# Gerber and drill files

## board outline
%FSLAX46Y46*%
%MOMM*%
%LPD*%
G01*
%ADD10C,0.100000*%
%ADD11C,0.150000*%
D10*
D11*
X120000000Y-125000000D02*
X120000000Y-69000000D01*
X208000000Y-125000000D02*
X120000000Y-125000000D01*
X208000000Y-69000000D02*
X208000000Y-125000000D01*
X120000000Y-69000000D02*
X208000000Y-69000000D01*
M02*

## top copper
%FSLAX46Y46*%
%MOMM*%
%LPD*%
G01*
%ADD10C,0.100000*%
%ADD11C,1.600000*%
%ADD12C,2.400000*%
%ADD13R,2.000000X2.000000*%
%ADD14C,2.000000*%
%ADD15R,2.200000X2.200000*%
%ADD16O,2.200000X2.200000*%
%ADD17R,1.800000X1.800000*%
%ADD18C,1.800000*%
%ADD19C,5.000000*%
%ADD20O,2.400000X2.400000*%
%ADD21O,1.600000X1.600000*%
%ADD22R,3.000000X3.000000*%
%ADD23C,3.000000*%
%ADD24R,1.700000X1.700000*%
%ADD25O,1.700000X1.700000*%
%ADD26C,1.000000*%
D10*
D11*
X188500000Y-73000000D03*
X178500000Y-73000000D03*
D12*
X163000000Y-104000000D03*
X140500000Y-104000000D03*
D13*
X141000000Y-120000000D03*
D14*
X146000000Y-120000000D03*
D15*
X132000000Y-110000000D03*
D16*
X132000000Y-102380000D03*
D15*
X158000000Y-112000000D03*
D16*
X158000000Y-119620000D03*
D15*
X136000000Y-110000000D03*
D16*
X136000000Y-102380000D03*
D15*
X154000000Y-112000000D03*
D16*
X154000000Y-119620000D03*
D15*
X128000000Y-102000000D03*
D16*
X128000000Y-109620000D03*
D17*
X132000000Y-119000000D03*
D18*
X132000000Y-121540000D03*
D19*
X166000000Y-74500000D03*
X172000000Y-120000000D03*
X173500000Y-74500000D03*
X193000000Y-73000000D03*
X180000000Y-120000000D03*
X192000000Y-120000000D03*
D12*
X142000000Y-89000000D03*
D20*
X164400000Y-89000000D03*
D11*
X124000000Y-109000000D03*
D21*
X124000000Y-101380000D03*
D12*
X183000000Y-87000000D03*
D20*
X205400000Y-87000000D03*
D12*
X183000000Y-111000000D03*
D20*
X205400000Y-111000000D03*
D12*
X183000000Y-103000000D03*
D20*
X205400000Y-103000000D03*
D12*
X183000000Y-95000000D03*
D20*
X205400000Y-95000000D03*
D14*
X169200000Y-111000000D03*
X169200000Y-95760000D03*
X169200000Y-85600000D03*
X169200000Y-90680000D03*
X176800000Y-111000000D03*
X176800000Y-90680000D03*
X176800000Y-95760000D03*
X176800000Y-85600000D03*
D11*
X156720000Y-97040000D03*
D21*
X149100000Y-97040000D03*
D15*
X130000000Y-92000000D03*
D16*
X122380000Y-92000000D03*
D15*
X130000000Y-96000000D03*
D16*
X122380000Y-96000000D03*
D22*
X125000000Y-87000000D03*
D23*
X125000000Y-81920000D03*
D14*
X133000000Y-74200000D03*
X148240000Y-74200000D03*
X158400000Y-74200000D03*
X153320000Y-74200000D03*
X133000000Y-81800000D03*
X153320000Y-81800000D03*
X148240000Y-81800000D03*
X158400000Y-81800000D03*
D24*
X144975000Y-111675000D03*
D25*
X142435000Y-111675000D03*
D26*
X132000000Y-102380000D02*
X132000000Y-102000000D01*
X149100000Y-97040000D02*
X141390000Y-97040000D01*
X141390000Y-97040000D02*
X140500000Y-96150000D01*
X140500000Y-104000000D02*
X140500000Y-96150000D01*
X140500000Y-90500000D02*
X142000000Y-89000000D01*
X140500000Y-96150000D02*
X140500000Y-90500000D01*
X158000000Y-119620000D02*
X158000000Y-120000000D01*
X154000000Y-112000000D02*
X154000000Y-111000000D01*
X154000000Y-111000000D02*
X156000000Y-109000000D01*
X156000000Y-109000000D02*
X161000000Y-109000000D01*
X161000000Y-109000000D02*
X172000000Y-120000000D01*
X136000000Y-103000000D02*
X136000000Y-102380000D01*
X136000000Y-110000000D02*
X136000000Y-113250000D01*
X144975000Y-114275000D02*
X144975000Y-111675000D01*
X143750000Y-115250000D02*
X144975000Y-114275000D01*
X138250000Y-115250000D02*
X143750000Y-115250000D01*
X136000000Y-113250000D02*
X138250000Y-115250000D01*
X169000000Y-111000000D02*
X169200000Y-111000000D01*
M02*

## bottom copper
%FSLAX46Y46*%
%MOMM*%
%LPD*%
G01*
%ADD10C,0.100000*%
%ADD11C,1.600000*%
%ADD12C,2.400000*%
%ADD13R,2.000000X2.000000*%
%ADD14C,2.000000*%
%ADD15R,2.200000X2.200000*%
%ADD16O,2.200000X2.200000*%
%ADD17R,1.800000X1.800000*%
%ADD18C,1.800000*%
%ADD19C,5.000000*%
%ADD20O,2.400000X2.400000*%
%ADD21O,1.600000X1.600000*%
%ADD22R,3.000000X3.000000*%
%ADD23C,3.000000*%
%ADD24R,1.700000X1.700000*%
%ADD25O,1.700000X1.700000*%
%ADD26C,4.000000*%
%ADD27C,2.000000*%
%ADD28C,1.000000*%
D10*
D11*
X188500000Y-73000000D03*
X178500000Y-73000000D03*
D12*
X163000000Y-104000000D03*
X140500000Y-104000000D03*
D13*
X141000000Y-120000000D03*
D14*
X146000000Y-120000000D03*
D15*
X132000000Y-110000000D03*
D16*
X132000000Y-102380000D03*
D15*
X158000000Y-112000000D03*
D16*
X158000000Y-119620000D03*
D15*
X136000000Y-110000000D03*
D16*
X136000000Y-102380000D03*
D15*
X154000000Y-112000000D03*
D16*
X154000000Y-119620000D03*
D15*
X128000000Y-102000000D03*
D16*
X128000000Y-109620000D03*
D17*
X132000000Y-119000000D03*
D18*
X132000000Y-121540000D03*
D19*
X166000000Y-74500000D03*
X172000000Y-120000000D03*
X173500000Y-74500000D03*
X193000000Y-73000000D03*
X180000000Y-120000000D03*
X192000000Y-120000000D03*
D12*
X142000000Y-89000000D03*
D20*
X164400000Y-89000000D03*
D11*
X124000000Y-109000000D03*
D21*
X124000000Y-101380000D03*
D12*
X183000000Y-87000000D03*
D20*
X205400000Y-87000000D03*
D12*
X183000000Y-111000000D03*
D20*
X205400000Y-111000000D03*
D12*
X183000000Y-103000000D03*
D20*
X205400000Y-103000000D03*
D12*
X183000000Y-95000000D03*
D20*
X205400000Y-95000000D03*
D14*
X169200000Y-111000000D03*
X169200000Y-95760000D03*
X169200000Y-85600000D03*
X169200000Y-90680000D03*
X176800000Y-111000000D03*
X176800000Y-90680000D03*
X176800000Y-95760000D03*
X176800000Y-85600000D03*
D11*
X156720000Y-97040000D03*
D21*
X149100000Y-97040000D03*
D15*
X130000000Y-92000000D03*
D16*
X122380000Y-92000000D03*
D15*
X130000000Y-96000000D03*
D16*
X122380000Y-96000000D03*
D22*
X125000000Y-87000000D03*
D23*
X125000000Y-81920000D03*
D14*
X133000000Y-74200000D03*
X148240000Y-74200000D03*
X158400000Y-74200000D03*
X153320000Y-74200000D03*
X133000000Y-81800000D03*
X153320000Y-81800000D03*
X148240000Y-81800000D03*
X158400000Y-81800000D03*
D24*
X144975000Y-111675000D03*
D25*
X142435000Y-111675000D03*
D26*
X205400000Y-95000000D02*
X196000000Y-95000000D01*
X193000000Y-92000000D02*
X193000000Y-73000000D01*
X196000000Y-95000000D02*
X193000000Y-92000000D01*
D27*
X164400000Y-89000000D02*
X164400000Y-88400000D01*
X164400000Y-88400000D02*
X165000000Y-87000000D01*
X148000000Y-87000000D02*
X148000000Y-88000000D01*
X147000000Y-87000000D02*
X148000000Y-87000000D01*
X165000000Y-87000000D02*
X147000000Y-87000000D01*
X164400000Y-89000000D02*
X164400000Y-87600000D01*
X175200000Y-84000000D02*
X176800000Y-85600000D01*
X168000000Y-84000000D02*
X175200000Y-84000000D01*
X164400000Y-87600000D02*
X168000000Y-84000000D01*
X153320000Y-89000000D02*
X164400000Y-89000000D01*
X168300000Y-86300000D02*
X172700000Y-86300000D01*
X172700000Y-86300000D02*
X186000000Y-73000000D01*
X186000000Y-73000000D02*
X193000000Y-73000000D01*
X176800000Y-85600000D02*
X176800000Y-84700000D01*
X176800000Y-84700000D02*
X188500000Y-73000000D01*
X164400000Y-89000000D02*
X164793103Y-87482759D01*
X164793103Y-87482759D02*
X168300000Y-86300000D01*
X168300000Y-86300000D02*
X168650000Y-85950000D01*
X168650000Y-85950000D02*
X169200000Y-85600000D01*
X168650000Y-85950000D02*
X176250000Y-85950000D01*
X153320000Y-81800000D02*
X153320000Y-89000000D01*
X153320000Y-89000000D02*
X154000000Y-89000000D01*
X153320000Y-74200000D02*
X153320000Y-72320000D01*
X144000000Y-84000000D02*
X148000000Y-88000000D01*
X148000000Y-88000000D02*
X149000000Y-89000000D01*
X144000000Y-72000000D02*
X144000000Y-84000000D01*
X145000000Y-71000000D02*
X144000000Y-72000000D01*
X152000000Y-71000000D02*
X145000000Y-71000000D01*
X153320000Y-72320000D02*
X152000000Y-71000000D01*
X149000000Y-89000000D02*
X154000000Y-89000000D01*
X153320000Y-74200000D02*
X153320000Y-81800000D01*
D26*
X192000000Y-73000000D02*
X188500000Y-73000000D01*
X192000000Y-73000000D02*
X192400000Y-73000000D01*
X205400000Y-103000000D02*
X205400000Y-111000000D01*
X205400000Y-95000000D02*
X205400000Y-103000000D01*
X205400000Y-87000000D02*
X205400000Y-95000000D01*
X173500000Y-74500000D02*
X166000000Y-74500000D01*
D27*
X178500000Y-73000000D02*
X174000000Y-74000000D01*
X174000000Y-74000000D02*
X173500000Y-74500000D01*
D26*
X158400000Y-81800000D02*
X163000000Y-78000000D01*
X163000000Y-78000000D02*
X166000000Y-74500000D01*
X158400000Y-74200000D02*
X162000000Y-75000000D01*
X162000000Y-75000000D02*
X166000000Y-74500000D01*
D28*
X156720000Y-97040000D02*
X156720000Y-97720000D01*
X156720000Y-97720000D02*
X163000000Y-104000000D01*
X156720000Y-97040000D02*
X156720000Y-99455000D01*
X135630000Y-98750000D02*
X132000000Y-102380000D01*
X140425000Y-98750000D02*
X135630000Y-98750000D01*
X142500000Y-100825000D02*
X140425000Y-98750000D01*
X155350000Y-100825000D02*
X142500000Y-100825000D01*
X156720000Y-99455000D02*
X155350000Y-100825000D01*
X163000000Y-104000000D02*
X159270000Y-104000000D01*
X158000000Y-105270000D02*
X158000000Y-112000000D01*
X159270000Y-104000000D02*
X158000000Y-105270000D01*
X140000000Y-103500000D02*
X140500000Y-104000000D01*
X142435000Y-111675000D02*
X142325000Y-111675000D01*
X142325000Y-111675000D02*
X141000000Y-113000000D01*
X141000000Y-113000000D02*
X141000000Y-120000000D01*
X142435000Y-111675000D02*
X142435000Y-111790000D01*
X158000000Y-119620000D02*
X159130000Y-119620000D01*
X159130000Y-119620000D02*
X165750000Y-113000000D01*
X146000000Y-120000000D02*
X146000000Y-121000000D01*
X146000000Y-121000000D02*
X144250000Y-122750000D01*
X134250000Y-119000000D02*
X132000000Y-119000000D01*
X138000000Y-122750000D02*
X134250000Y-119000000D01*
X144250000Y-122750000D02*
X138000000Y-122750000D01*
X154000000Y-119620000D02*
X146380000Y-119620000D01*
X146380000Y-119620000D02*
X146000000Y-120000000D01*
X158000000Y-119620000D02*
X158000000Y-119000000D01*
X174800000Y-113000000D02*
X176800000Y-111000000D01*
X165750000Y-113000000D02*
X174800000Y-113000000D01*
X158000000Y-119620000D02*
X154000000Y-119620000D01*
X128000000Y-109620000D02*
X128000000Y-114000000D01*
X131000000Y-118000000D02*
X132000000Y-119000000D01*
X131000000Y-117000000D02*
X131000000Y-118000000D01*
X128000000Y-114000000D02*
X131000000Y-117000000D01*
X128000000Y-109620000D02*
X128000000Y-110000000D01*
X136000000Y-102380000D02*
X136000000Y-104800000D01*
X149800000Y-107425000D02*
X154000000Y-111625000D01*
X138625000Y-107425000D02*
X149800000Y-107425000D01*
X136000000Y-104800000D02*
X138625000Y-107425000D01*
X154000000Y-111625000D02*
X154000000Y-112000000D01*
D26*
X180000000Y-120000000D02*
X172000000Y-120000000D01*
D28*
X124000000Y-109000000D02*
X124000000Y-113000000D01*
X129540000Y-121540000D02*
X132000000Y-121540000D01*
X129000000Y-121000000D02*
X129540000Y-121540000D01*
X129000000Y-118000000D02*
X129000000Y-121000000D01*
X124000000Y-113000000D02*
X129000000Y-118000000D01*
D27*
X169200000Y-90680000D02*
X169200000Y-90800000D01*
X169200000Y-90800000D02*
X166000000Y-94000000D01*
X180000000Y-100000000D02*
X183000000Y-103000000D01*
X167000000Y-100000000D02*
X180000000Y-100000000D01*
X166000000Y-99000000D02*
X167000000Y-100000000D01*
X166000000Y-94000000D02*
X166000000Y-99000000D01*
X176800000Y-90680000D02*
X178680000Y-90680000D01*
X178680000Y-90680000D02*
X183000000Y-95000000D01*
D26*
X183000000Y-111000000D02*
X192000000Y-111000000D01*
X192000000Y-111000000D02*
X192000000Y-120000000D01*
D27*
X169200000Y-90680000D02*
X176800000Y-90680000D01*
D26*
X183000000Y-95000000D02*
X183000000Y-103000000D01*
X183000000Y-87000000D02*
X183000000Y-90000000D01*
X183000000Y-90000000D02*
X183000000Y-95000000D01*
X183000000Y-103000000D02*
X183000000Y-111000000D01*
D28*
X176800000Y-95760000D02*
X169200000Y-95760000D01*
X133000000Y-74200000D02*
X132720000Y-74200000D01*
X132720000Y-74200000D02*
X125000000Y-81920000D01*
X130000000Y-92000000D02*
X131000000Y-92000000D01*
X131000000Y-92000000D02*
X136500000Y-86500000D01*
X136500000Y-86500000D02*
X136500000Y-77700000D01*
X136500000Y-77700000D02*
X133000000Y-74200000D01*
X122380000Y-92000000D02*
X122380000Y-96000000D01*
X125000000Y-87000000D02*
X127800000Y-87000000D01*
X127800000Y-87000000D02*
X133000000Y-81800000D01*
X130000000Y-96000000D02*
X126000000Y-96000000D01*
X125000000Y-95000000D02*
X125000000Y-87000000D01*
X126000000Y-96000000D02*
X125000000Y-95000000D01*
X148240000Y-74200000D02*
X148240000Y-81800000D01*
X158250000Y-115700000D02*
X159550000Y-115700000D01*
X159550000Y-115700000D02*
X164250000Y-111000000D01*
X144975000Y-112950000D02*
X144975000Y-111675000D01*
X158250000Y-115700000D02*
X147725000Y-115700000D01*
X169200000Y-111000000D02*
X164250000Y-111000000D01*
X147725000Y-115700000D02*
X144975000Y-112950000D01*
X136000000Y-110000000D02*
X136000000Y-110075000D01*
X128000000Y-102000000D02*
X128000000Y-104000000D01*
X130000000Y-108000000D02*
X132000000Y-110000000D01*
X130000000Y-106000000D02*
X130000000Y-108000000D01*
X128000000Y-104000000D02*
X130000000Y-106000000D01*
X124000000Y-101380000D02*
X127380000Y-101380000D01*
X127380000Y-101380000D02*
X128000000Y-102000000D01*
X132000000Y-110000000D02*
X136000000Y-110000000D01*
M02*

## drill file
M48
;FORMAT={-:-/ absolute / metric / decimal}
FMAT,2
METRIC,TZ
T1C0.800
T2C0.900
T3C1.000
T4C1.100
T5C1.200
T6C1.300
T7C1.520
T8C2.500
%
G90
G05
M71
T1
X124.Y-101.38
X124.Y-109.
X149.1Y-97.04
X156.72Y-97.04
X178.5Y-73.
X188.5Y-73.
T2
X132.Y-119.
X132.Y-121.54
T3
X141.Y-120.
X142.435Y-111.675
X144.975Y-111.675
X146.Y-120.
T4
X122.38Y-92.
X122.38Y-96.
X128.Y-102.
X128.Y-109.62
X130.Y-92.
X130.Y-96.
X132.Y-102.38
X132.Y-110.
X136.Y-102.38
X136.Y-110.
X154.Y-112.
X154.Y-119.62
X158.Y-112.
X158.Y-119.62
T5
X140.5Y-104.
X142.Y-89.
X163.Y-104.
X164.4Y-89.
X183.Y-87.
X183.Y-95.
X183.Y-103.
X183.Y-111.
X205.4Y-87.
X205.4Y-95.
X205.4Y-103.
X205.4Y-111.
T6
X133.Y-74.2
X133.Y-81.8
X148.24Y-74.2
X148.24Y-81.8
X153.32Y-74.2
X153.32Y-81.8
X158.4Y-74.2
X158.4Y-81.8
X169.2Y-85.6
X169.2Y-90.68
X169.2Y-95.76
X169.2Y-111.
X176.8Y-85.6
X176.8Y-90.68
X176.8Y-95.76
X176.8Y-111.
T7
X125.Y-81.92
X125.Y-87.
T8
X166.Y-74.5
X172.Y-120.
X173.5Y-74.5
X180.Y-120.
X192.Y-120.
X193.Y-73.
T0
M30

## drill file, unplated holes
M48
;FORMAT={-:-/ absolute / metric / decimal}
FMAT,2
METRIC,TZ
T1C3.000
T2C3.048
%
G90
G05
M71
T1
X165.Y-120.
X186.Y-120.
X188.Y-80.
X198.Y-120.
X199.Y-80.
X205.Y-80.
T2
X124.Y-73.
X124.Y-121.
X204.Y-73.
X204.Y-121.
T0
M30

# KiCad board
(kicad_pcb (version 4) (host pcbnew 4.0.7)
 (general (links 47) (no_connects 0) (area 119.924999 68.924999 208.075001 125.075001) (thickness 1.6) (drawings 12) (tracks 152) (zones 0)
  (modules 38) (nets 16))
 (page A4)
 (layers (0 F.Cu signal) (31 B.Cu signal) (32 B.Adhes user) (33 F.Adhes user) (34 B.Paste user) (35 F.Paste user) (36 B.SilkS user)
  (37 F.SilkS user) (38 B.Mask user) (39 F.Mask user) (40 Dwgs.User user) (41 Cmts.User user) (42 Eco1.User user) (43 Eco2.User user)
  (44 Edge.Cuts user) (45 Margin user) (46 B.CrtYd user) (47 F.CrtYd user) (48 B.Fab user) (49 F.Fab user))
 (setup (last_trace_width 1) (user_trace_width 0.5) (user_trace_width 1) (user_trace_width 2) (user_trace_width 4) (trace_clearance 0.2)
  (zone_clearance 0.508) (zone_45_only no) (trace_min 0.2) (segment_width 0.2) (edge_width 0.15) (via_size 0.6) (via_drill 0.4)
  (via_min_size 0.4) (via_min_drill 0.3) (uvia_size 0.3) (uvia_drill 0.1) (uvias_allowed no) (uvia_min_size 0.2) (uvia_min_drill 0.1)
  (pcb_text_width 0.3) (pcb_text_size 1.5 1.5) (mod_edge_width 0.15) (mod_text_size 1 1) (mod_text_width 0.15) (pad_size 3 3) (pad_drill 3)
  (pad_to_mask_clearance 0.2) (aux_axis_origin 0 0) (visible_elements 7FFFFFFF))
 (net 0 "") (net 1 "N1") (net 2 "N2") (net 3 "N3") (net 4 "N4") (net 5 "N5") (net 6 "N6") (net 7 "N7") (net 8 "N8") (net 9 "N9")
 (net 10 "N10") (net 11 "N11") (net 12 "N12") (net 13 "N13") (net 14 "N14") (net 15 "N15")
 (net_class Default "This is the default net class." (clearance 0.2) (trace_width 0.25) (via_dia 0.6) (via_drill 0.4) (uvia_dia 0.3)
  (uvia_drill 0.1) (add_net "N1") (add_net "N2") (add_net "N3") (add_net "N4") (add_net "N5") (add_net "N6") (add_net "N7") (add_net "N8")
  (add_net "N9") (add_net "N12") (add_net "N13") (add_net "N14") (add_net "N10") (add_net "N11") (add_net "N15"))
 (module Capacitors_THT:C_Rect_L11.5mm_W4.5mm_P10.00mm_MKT (layer F.Cu) (at 188.5 73 180)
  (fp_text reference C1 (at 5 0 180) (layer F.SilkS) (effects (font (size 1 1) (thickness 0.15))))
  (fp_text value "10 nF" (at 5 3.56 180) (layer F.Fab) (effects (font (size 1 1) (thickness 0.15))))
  (pad 1 thru_hole circle (at 0 0 180) (size 1.6 1.6) (drill 0.8) (layers *.Cu *.Mask) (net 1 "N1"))
  (pad 2 thru_hole circle (at 10 0 180) (size 1.6 1.6) (drill 0.8) (layers *.Cu *.Mask) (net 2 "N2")))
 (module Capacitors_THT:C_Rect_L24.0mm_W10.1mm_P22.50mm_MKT (layer F.Cu) (at 163 104 180)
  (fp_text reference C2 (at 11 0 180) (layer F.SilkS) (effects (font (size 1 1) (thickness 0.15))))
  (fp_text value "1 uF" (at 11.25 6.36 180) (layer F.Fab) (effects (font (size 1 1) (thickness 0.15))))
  (pad 1 thru_hole circle (at 0 0 180) (size 2.4 2.4) (drill 1.2) (layers *.Cu *.Mask) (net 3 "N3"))
  (pad 2 thru_hole circle (at 22.5 0 180) (size 2.4 2.4) (drill 1.2) (layers *.Cu *.Mask) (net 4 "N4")))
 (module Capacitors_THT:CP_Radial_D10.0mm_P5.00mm (layer F.Cu) (at 141 120)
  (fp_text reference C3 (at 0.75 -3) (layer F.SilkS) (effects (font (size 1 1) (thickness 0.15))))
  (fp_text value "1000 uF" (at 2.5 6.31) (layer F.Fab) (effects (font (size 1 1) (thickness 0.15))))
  (pad 1 thru_hole rect (at 0 0) (size 2 2) (drill 1) (layers *.Cu *.Mask) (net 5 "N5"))
  (pad 2 thru_hole circle (at 5 0) (size 2 2) (drill 1) (layers *.Cu *.Mask) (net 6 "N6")))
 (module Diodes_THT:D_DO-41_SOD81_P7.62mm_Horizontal (layer F.Cu) (at 132 110 90)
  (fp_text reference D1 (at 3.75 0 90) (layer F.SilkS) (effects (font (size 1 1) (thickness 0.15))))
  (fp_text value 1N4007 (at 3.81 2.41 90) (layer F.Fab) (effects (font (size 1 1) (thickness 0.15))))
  (pad 1 thru_hole rect (at 0 0 90) (size 2.2 2.2) (drill 1.1) (layers *.Cu *.Mask) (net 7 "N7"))
  (pad 2 thru_hole oval (at 7.62 0 90) (size 2.2 2.2) (drill 1.1) (layers *.Cu *.Mask) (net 3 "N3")))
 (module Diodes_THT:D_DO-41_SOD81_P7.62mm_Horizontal (layer F.Cu) (at 158 112 270)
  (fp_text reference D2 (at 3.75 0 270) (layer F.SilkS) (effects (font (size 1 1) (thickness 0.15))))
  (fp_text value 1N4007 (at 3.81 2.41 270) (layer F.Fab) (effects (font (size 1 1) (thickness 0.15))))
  (pad 1 thru_hole rect (at 0 0 270) (size 2.2 2.2) (drill 1.1) (layers *.Cu *.Mask) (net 3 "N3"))
  (pad 2 thru_hole oval (at 7.62 0 270) (size 2.2 2.2) (drill 1.1) (layers *.Cu *.Mask) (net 6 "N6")))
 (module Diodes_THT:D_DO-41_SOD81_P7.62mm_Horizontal (layer F.Cu) (at 136 110 90)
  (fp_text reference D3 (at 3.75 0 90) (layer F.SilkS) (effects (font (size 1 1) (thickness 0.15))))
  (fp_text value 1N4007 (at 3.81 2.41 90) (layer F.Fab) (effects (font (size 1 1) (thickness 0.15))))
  (pad 1 thru_hole rect (at 0 0 90) (size 2.2 2.2) (drill 1.1) (layers *.Cu *.Mask) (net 7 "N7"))
  (pad 2 thru_hole oval (at 7.62 0 90) (size 2.2 2.2) (drill 1.1) (layers *.Cu *.Mask) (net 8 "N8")))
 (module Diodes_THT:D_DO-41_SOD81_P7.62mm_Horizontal (layer F.Cu) (at 154 112 270)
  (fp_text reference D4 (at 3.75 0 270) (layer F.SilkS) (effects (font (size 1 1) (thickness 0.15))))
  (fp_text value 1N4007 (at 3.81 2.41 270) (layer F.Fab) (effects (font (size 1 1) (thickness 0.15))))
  (pad 1 thru_hole rect (at 0 0 270) (size 2.2 2.2) (drill 1.1) (layers *.Cu *.Mask) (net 8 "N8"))
  (pad 2 thru_hole oval (at 7.62 0 270) (size 2.2 2.2) (drill 1.1) (layers *.Cu *.Mask) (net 6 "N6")))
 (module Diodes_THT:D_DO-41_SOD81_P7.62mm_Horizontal (layer F.Cu) (at 128 102 270)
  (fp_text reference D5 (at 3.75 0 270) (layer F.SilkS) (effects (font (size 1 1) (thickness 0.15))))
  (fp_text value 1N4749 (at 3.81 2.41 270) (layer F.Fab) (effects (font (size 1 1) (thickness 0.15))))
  (pad 1 thru_hole rect (at 0 0 270) (size 2.2 2.2) (drill 1.1) (layers *.Cu *.Mask) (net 7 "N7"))
  (pad 2 thru_hole oval (at 7.62 0 270) (size 2.2 2.2) (drill 1.1) (layers *.Cu *.Mask) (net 6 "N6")))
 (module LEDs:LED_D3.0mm (layer F.Cu) (at 132 119 270)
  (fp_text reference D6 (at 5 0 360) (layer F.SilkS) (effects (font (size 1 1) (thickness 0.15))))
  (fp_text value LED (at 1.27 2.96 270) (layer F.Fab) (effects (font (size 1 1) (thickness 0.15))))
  (pad 1 thru_hole rect (at 0 0 270) (size 1.8 1.8) (drill 0.9) (layers *.Cu *.Mask) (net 6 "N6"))
  (pad 2 thru_hole circle (at 2.54 0 270) (size 1.8 1.8) (drill 0.9) (layers *.Cu *.Mask) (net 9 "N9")))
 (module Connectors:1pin (layer F.Cu) (at 166 74.5)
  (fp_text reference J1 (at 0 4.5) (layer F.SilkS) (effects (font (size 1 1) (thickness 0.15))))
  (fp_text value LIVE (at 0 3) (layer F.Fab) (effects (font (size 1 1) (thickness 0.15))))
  (pad 1 thru_hole circle (at 0 0) (size 5 5) (drill 2.5) (layers *.Cu *.Mask) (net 2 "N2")))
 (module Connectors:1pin (layer F.Cu) (at 172 120)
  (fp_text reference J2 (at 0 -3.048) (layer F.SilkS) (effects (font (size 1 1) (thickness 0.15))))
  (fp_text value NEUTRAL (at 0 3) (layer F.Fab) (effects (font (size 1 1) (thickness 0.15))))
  (pad 1 thru_hole circle (at 0 0) (size 5 5) (drill 2.5) (layers *.Cu *.Mask) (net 8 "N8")))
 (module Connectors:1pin (layer F.Cu) (at 173.5 74.5)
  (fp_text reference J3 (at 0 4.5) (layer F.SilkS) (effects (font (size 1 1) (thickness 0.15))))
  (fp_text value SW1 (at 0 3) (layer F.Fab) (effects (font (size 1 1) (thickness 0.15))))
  (pad 1 thru_hole circle (at 0 0) (size 5 5) (drill 2.5) (layers *.Cu *.Mask) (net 2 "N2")))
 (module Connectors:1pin (layer F.Cu) (at 193 73)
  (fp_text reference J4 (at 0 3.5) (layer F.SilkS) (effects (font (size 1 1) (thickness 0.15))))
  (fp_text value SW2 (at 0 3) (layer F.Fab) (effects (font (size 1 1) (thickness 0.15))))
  (pad 1 thru_hole circle (at 0 0) (size 5 5) (drill 2.5) (layers *.Cu *.Mask) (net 1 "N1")))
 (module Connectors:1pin (layer F.Cu) (at 180 120)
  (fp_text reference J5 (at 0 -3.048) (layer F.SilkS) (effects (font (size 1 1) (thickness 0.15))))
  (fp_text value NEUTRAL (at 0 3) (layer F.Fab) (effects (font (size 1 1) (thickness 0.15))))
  (pad 1 thru_hole circle (at 0 0) (size 5 5) (drill 2.5) (layers *.Cu *.Mask) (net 8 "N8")))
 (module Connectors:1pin (layer F.Cu) (at 192 120)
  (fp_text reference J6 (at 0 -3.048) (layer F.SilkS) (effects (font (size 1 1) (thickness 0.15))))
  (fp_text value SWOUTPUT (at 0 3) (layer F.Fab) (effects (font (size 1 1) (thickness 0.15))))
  (pad 1 thru_hole circle (at 0 0) (size 5 5) (drill 2.5) (layers *.Cu *.Mask) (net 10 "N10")))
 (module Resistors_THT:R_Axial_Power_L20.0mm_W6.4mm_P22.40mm (layer F.Cu) (at 142 89)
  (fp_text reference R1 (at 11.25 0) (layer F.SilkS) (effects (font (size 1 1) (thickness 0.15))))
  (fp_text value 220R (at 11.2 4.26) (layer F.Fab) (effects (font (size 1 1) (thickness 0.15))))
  (pad 1 thru_hole circle (at 0 0) (size 2.4 2.4) (drill 1.2) (layers *.Cu *.Mask) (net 4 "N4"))
  (pad 2 thru_hole oval (at 22.4 0) (size 2.4 2.4) (drill 1.2) (layers *.Cu *.Mask) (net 1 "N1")))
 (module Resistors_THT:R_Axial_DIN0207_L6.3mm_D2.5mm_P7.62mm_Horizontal (layer F.Cu) (at 124 109 90)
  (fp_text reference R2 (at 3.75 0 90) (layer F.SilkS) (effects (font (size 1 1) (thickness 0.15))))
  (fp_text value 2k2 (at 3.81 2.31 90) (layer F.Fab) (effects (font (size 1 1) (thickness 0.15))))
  (pad 1 thru_hole circle (at 0 0 90) (size 1.6 1.6) (drill 0.8) (layers *.Cu *.Mask) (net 9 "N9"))
  (pad 2 thru_hole oval (at 7.62 0 90) (size 1.6 1.6) (drill 0.8) (layers *.Cu *.Mask) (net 7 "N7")))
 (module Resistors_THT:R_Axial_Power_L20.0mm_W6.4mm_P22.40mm (layer F.Cu) (at 183 87)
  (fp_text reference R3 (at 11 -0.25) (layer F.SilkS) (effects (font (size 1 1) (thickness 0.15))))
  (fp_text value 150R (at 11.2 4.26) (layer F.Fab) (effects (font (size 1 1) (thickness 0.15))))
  (pad 1 thru_hole circle (at 0 0) (size 2.4 2.4) (drill 1.2) (layers *.Cu *.Mask) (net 10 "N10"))
  (pad 2 thru_hole oval (at 22.4 0) (size 2.4 2.4) (drill 1.2) (layers *.Cu *.Mask) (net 1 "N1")))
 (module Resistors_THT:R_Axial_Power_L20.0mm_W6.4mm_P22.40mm (layer F.Cu) (at 183 111)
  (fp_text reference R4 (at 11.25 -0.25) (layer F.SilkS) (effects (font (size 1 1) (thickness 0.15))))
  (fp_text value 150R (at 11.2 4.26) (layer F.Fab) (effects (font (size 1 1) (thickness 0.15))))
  (pad 1 thru_hole circle (at 0 0) (size 2.4 2.4) (drill 1.2) (layers *.Cu *.Mask) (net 10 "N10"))
  (pad 2 thru_hole oval (at 22.4 0) (size 2.4 2.4) (drill 1.2) (layers *.Cu *.Mask) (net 1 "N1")))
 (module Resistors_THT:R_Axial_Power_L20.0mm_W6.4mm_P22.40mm (layer F.Cu) (at 183 103)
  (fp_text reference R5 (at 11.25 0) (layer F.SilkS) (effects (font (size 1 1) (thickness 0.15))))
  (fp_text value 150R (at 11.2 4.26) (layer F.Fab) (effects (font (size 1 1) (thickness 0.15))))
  (pad 1 thru_hole circle (at 0 0) (size 2.4 2.4) (drill 1.2) (layers *.Cu *.Mask) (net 10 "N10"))
  (pad 2 thru_hole oval (at 22.4 0) (size 2.4 2.4) (drill 1.2) (layers *.Cu *.Mask) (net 1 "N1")))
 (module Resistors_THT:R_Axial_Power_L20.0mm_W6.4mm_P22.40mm (layer F.Cu) (at 183 95)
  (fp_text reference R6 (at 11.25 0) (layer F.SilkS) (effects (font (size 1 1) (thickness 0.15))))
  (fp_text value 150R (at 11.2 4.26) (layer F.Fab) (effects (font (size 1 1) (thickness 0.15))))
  (pad 1 thru_hole circle (at 0 0) (size 2.4 2.4) (drill 1.2) (layers *.Cu *.Mask) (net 10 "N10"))
  (pad 2 thru_hole oval (at 22.4 0) (size 2.4 2.4) (drill 1.2) (layers *.Cu *.Mask) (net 1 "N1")))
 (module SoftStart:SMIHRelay (layer F.Cu) (at 173 101 90)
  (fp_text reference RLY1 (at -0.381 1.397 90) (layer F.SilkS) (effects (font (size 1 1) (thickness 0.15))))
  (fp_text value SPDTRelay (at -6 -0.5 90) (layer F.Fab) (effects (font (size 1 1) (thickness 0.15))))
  (pad 4 thru_hole circle (at -10 -3.8 90) (size 2 2) (drill 1.3) (layers *.Cu *.Mask) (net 7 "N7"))
  (pad 2 thru_hole circle (at 5.24 -3.8 90) (size 2 2) (drill 1.3) (layers *.Cu *.Mask) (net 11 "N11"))
  (pad 3 thru_hole circle (at 15.4 -3.8 90) (size 2 2) (drill 1.3) (layers *.Cu *.Mask) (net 1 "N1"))
  (pad 1 thru_hole circle (at 10.32 -3.8 90) (size 2 2) (drill 1.3) (layers *.Cu *.Mask) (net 10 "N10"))
  (pad 5 thru_hole circle (at -10 3.8 90) (size 2 2) (drill 1.3) (layers *.Cu *.Mask) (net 6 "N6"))
  (pad 1 thru_hole circle (at 10.32 3.8 90) (size 2 2) (drill 1.3) (layers *.Cu *.Mask) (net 10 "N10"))
  (pad 2 thru_hole circle (at 5.24 3.8 90) (size 2 2) (drill 1.3) (layers *.Cu *.Mask) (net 11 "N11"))
  (pad 3 thru_hole circle (at 15.4 3.8 90) (size 2 2) (drill 1.3) (layers *.Cu *.Mask) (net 1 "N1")))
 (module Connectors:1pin (layer F.Cu) (at 204 121)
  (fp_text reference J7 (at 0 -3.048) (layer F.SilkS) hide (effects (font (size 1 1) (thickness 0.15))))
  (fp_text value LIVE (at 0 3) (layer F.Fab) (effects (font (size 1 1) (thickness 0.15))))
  (pad "" np_thru_hole circle (at 0 0) (size 3.048 3.048) (drill 3.048) (layers *.Cu *.Mask)))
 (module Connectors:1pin (layer F.Cu) (at 204 73)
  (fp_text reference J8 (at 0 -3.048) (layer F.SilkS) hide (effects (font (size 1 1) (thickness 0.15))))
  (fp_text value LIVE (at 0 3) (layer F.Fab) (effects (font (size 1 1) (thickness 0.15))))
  (pad "" np_thru_hole circle (at 0 0) (size 3.048 3.048) (drill 3.048) (layers *.Cu *.Mask)))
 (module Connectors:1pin (layer F.Cu) (at 124 73)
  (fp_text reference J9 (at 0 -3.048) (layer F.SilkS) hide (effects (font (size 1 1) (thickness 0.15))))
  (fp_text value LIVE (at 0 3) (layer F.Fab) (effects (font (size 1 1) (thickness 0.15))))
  (pad "" np_thru_hole circle (at 0 0) (size 3.048 3.048) (drill 3.048) (layers *.Cu *.Mask)))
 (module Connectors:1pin (layer F.Cu) (at 124 121)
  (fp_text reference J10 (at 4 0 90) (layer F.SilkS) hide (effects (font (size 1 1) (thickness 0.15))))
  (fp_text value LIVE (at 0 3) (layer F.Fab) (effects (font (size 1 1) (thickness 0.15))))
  (pad "" np_thru_hole circle (at 0 0) (size 3.048 3.048) (drill 3.048) (layers *.Cu *.Mask)))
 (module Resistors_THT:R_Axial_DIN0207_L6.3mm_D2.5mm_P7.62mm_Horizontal (layer F.Cu) (at 156.72 97.04 180)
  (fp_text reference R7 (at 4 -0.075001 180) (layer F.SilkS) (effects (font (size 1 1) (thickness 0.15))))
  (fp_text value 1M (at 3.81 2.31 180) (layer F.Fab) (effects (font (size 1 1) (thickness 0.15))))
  (pad 1 thru_hole circle (at 0 0 180) (size 1.6 1.6) (drill 0.8) (layers *.Cu *.Mask) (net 3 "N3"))
  (pad 2 thru_hole oval (at 7.62 0 180) (size 1.6 1.6) (drill 0.8) (layers *.Cu *.Mask) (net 4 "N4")))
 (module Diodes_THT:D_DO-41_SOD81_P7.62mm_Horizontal (layer F.Cu) (at 130 92 180)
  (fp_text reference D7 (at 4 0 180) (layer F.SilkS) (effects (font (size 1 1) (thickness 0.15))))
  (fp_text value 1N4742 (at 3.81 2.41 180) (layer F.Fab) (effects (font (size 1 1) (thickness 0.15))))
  (pad 1 thru_hole rect (at 0 0 180) (size 2.2 2.2) (drill 1.1) (layers *.Cu *.Mask) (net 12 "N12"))
  (pad 2 thru_hole oval (at 7.62 0 180) (size 2.2 2.2) (drill 1.1) (layers *.Cu *.Mask) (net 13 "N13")))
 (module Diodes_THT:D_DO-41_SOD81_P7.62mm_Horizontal (layer F.Cu) (at 130 96 180)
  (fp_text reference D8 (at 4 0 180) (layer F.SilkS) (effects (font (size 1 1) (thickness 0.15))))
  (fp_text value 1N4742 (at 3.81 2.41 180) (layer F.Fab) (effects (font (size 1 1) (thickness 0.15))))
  (pad 1 thru_hole rect (at 0 0 180) (size 2.2 2.2) (drill 1.1) (layers *.Cu *.Mask) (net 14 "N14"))
  (pad 2 thru_hole oval (at 7.62 0 180) (size 2.2 2.2) (drill 1.1) (layers *.Cu *.Mask) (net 13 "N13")))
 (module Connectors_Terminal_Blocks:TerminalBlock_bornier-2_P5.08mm (layer F.Cu) (at 125 87 90)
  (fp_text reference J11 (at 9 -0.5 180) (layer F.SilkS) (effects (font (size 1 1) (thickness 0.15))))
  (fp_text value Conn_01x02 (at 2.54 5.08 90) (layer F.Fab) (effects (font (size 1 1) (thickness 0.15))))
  (pad 1 thru_hole rect (at 0 0 90) (size 3 3) (drill 1.52) (layers *.Cu *.Mask) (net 14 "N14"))
  (pad 2 thru_hole circle (at 5.08 0 90) (size 3 3) (drill 1.52) (layers *.Cu *.Mask) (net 12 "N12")))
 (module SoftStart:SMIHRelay (layer F.Cu) (at 143 78)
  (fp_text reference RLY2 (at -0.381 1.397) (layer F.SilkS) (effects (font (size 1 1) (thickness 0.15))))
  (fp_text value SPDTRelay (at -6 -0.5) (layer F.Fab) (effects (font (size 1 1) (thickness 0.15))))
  (pad 4 thru_hole circle (at -10 -3.8) (size 2 2) (drill 1.3) (layers *.Cu *.Mask) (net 12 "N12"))
  (pad 2 thru_hole circle (at 5.24 -3.8) (size 2 2) (drill 1.3) (layers *.Cu *.Mask) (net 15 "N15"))
  (pad 3 thru_hole circle (at 15.4 -3.8) (size 2 2) (drill 1.3) (layers *.Cu *.Mask) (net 2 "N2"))
  (pad 1 thru_hole circle (at 10.32 -3.8) (size 2 2) (drill 1.3) (layers *.Cu *.Mask) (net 1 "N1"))
  (pad 5 thru_hole circle (at -10 3.8) (size 2 2) (drill 1.3) (layers *.Cu *.Mask) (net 14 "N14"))
  (pad 1 thru_hole circle (at 10.32 3.8) (size 2 2) (drill 1.3) (layers *.Cu *.Mask) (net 1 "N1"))
  (pad 2 thru_hole circle (at 5.24 3.8) (size 2 2) (drill 1.3) (layers *.Cu *.Mask) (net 15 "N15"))
  (pad 3 thru_hole circle (at 15.4 3.8) (size 2 2) (drill 1.3) (layers *.Cu *.Mask) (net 2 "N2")))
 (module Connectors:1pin (layer F.Cu) (at 188 80)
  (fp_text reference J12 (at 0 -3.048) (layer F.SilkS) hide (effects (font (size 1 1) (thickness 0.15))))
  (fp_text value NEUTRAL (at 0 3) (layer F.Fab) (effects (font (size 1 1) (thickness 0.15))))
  (pad "" np_thru_hole circle (at 0 0) (size 3 3) (drill 3) (layers *.Cu *.Mask)))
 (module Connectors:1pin (layer F.Cu) (at 199 80)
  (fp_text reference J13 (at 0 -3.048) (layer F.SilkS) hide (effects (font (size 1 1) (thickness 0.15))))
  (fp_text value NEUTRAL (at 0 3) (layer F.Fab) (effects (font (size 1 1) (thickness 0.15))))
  (pad "" np_thru_hole circle (at 0 0) (size 3 3) (drill 3) (layers *.Cu *.Mask)))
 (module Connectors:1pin (layer F.Cu) (at 205 80)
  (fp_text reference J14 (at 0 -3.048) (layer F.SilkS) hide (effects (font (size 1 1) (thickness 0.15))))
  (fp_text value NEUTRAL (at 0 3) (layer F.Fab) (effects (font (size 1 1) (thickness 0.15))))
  (pad "" np_thru_hole circle (at 0 0) (size 3 3) (drill 3) (layers *.Cu *.Mask)))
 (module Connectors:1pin (layer F.Cu) (at 186 120)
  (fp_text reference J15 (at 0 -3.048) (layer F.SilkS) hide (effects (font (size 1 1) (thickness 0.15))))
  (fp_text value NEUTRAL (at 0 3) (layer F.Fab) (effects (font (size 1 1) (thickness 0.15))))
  (pad "" np_thru_hole circle (at 0 0) (size 3 3) (drill 3) (layers *.Cu *.Mask)))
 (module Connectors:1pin (layer F.Cu) (at 198 120)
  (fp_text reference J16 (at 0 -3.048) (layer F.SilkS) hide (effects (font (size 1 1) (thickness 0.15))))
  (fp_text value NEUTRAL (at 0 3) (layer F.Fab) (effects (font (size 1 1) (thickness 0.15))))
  (pad "" np_thru_hole circle (at 0 0) (size 3 3) (drill 3) (layers *.Cu *.Mask)))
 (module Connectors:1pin (layer F.Cu) (at 165 120)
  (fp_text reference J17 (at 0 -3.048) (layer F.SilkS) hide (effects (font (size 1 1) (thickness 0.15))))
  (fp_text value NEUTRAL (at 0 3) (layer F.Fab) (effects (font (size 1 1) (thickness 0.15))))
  (pad "" np_thru_hole circle (at 0 0) (size 3 3) (drill 3) (layers *.Cu *.Mask)))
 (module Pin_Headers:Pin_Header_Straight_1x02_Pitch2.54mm (layer F.Cu) (at 144.975 111.675 270)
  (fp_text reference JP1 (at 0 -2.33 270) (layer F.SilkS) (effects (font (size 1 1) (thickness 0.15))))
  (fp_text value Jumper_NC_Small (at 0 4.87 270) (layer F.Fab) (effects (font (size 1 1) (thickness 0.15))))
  (pad 1 thru_hole rect (at 0 0 270) (size 1.7 1.7) (drill 1) (layers *.Cu *.Mask) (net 7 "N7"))
  (pad 2 thru_hole oval (at 0 2.54 270) (size 1.7 1.7) (drill 1) (layers *.Cu *.Mask) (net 5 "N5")))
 (gr_line (start 120 125) (end 120 69) (angle 90) (layer Edge.Cuts) (width 0.15))
 (gr_line (start 208 125) (end 120 125) (angle 90) (layer Edge.Cuts) (width 0.15))
 (gr_line (start 208 69) (end 208 125) (angle 90) (layer Edge.Cuts) (width 0.15))
 (gr_line (start 120 69) (end 208 69) (angle 90) (layer Edge.Cuts) (width 0.15))
 (segment (start 205.4 95) (end 196 95) (width 4) (layer B.Cu) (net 1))
 (segment (start 193 92) (end 193 73) (width 4) (layer B.Cu) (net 1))
 (segment (start 196 95) (end 193 92) (width 4) (layer B.Cu) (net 1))
 (segment (start 164.4 89) (end 164.4 88.4) (width 2) (layer B.Cu) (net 1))
 (segment (start 164.4 88.4) (end 165 87) (width 2) (layer B.Cu) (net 1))
 (segment (start 148 87) (end 148 88) (width 2) (layer B.Cu) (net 1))
 (segment (start 147 87) (end 148 87) (width 2) (layer B.Cu) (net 1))
 (segment (start 165 87) (end 147 87) (width 2) (layer B.Cu) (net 1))
 (segment (start 164.4 89) (end 164.4 87.6) (width 2) (layer B.Cu) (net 1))
 (segment (start 175.2 84) (end 176.8 85.6) (width 2) (layer B.Cu) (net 1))
 (segment (start 168 84) (end 175.2 84) (width 2) (layer B.Cu) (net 1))
 (segment (start 164.4 87.6) (end 168 84) (width 2) (layer B.Cu) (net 1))
 (segment (start 153.32 89) (end 164.4 89) (width 2) (layer B.Cu) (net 1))
 (segment (start 168.3 86.3) (end 172.7 86.3) (width 2) (layer B.Cu) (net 1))
 (segment (start 172.7 86.3) (end 186 73) (width 2) (layer B.Cu) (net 1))
 (segment (start 186 73) (end 193 73) (width 2) (layer B.Cu) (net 1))
 (segment (start 176.8 85.6) (end 176.8 84.7) (width 2) (layer B.Cu) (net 1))
 (segment (start 176.8 84.7) (end 188.5 73) (width 2) (layer B.Cu) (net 1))
 (segment (start 164.4 89) (end 164.793103 87.482759) (width 2) (layer B.Cu) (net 1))
 (segment (start 164.793103 87.482759) (end 168.3 86.3) (width 2) (layer B.Cu) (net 1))
 (segment (start 168.3 86.3) (end 168.65 85.95) (width 2) (layer B.Cu) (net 1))
 (segment (start 168.65 85.95) (end 169.2 85.6) (width 2) (layer B.Cu) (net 1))
 (segment (start 168.65 85.95) (end 176.25 85.95) (width 2) (layer B.Cu) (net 1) (status 30))
 (segment (start 153.32 81.8) (end 153.32 89) (width 2) (layer B.Cu) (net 1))
 (segment (start 153.32 89) (end 154 89) (width 2) (layer B.Cu) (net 1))
 (segment (start 153.32 74.2) (end 153.32 72.32) (width 2) (layer B.Cu) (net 1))
 (segment (start 144 84) (end 148 88) (width 2) (layer B.Cu) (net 1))
 (segment (start 148 88) (end 149 89) (width 2) (layer B.Cu) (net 1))
 (segment (start 144 72) (end 144 84) (width 2) (layer B.Cu) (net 1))
 (segment (start 145 71) (end 144 72) (width 2) (layer B.Cu) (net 1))
 (segment (start 152 71) (end 145 71) (width 2) (layer B.Cu) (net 1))
 (segment (start 153.32 72.32) (end 152 71) (width 2) (layer B.Cu) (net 1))
 (segment (start 149 89) (end 154 89) (width 2) (layer B.Cu) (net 1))
 (segment (start 153.32 74.2) (end 153.32 81.8) (width 2) (layer B.Cu) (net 1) (status 30))
 (segment (start 192 73) (end 188.5 73) (width 4) (layer B.Cu) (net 1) (status 20))
 (segment (start 192 73) (end 192.4 73) (width 4) (layer B.Cu) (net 1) (status 30))
 (segment (start 205.4 103) (end 205.4 111) (width 4) (layer B.Cu) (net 1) (status 10))
 (segment (start 205.4 95) (end 205.4 103) (width 4) (layer B.Cu) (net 1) (status 10))
 (segment (start 205.4 87) (end 205.4 95) (width 4) (layer B.Cu) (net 1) (status 10))
 (segment (start 173.5 74.5) (end 166 74.5) (width 4) (layer B.Cu) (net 2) (status 10))
 (segment (start 178.5 73) (end 174 74) (width 2) (layer B.Cu) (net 2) (status 10))
 (segment (start 174 74) (end 173.5 74.5) (width 2) (layer B.Cu) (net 2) (status 30))
 (segment (start 158.4 81.8) (end 163 78) (width 4) (layer B.Cu) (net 2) (status 10))
 (segment (start 163 78) (end 166 74.5) (width 4) (layer B.Cu) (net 2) (status 20))
 (segment (start 158.4 74.2) (end 162 75) (width 4) (layer B.Cu) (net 2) (status 10))
 (segment (start 162 75) (end 166 74.5) (width 4) (layer B.Cu) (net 2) (status 20))
 (segment (start 156.72 97.04) (end 156.72 97.72) (width 1) (layer B.Cu) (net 3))
 (segment (start 156.72 97.72) (end 163 104) (width 1) (layer B.Cu) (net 3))
 (segment (start 156.72 97.04) (end 156.72 99.455) (width 1) (layer B.Cu) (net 3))
 (segment (start 135.63 98.75) (end 132 102.38) (width 1) (layer B.Cu) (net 3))
 (segment (start 140.425 98.75) (end 135.63 98.75) (width 1) (layer B.Cu) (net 3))
 (segment (start 142.5 100.825) (end 140.425 98.75) (width 1) (layer B.Cu) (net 3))
 (segment (start 155.35 100.825) (end 142.5 100.825) (width 1) (layer B.Cu) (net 3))
 (segment (start 156.72 99.455) (end 155.35 100.825) (width 1) (layer B.Cu) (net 3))
 (segment (start 163 104) (end 159.27 104) (width 1) (layer B.Cu) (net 3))
 (segment (start 158 105.27) (end 158 112) (width 1) (layer B.Cu) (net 3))
 (segment (start 159.27 104) (end 158 105.27) (width 1) (layer B.Cu) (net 3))
 (segment (start 132 102.38) (end 132 102) (width 1) (layer F.Cu) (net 3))
 (segment (start 149.1 97.04) (end 141.39 97.04) (width 1) (layer F.Cu) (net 4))
 (segment (start 141.39 97.04) (end 140.5 96.15) (width 1) (layer F.Cu) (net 4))
 (segment (start 140.5 104) (end 140.5 96.15) (width 1) (layer F.Cu) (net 4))
 (segment (start 140.5 90.5) (end 142 89) (width 1) (layer F.Cu) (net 4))
 (segment (start 140.5 96.15) (end 140.5 90.5) (width 1) (layer F.Cu) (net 4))
 (segment (start 140 103.5) (end 140.5 104) (width 1) (layer B.Cu) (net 4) (status 30))
 (segment (start 142.435 111.675) (end 142.325 111.675) (width 1) (layer B.Cu) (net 5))
 (segment (start 142.325 111.675) (end 141 113) (width 1) (layer B.Cu) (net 5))
 (segment (start 141 113) (end 141 120) (width 1) (layer B.Cu) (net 5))
 (segment (start 142.435 111.675) (end 142.435 111.79) (width 1) (layer B.Cu) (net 5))
 (segment (start 158 119.62) (end 159.13 119.62) (width 1) (layer B.Cu) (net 6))
 (segment (start 159.13 119.62) (end 165.75 113) (width 1) (layer B.Cu) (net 6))
 (segment (start 146 120) (end 146 121) (width 1) (layer B.Cu) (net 6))
 (segment (start 146 121) (end 144.25 122.75) (width 1) (layer B.Cu) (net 6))
 (segment (start 134.25 119) (end 132 119) (width 1) (layer B.Cu) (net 6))
 (segment (start 138 122.75) (end 134.25 119) (width 1) (layer B.Cu) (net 6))
 (segment (start 144.25 122.75) (end 138 122.75) (width 1) (layer B.Cu) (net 6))
 (segment (start 154 119.62) (end 146.38 119.62) (width 1) (layer B.Cu) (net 6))
 (segment (start 146.38 119.62) (end 146 120) (width 1) (layer B.Cu) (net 6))
 (segment (start 158 119.62) (end 158 119) (width 1) (layer B.Cu) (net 6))
 (segment (start 174.8 113) (end 176.8 111) (width 1) (layer B.Cu) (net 6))
 (segment (start 165.75 113) (end 174.8 113) (width 1) (layer B.Cu) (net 6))
 (segment (start 158 119.62) (end 154 119.62) (width 1) (layer B.Cu) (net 6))
 (segment (start 128 109.62) (end 128 114) (width 1) (layer B.Cu) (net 6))
 (segment (start 131 118) (end 132 119) (width 1) (layer B.Cu) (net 6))
 (segment (start 131 117) (end 131 118) (width 1) (layer B.Cu) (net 6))
 (segment (start 128 114) (end 131 117) (width 1) (layer B.Cu) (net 6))
 (segment (start 128 109.62) (end 128 110) (width 1) (layer B.Cu) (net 6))
 (segment (start 158 119.62) (end 158 120) (width 1) (layer F.Cu) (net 6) (status 30))
 (segment (start 136 102.38) (end 136 104.8) (width 1) (layer B.Cu) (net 8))
 (segment (start 149.8 107.425) (end 154 111.625) (width 1) (layer B.Cu) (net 8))
 (segment (start 138.625 107.425) (end 149.8 107.425) (width 1) (layer B.Cu) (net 8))
 (segment (start 136 104.8) (end 138.625 107.425) (width 1) (layer B.Cu) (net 8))
 (segment (start 154 111.625) (end 154 112) (width 1) (layer B.Cu) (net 8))
 (segment (start 154 112) (end 154 111) (width 1) (layer F.Cu) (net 8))
 (segment (start 154 111) (end 156 109) (width 1) (layer F.Cu) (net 8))
 (segment (start 156 109) (end 161 109) (width 1) (layer F.Cu) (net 8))
 (segment (start 161 109) (end 172 120) (width 1) (layer F.Cu) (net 8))
 (segment (start 136 103) (end 136 102.38) (width 1) (layer F.Cu) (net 8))
 (segment (start 180 120) (end 172 120) (width 4) (layer B.Cu) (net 8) (status 10))
 (segment (start 124 109) (end 124 113) (width 1) (layer B.Cu) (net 9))
 (segment (start 129.54 121.54) (end 132 121.54) (width 1) (layer B.Cu) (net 9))
 (segment (start 129 121) (end 129.54 121.54) (width 1) (layer B.Cu) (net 9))
 (segment (start 129 118) (end 129 121) (width 1) (layer B.Cu) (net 9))
 (segment (start 124 113) (end 129 118) (width 1) (layer B.Cu) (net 9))
 (segment (start 169.2 90.68) (end 169.2 90.8) (width 2) (layer B.Cu) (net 10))
 (segment (start 169.2 90.8) (end 166 94) (width 2) (layer B.Cu) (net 10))
 (segment (start 180 100) (end 183 103) (width 2) (layer B.Cu) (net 10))
 (segment (start 167 100) (end 180 100) (width 2) (layer B.Cu) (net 10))
 (segment (start 166 99) (end 167 100) (width 2) (layer B.Cu) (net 10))
 (segment (start 166 94) (end 166 99) (width 2) (layer B.Cu) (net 10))
 (segment (start 176.8 90.68) (end 178.68 90.68) (width 2) (layer B.Cu) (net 10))
 (segment (start 178.68 90.68) (end 183 95) (width 2) (layer B.Cu) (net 10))
 (segment (start 183 111) (end 192 111) (width 4) (layer B.Cu) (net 10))
 (segment (start 192 111) (end 192 120) (width 4) (layer B.Cu) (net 10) (status 20))
 (segment (start 169.2 90.68) (end 176.8 90.68) (width 2) (layer B.Cu) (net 10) (status 30))
 (segment (start 183 95) (end 183 103) (width 4) (layer B.Cu) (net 10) (status 10))
 (segment (start 183 87) (end 183 90) (width 4) (layer B.Cu) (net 10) (status 10))
 (segment (start 183 90) (end 183 95) (width 4) (layer B.Cu) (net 10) (status 20))
 (segment (start 183 103) (end 183 111) (width 4) (layer B.Cu) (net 10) (status 10))
 (segment (start 176.8 95.76) (end 169.2 95.76) (width 1) (layer B.Cu) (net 11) (status 30))
 (segment (start 133 74.2) (end 132.72 74.2) (width 1) (layer B.Cu) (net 12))
 (segment (start 132.72 74.2) (end 125 81.92) (width 1) (layer B.Cu) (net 12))
 (segment (start 130 92) (end 131 92) (width 1) (layer B.Cu) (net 12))
 (segment (start 131 92) (end 136.5 86.5) (width 1) (layer B.Cu) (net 12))
 (segment (start 136.5 86.5) (end 136.5 77.7) (width 1) (layer B.Cu) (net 12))
 (segment (start 136.5 77.7) (end 133 74.2) (width 1) (layer B.Cu) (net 12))
 (segment (start 122.38 92) (end 122.38 96) (width 1) (layer B.Cu) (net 13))
 (segment (start 125 87) (end 127.8 87) (width 1) (layer B.Cu) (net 14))
 (segment (start 127.8 87) (end 133 81.8) (width 1) (layer B.Cu) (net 14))
 (segment (start 130 96) (end 126 96) (width 1) (layer B.Cu) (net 14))
 (segment (start 125 95) (end 125 87) (width 1) (layer B.Cu) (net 14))
 (segment (start 126 96) (end 125 95) (width 1) (layer B.Cu) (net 14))
 (segment (start 148.24 74.2) (end 148.24 81.8) (width 1) (layer B.Cu) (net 15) (status 30))
 (segment (start 158.25 115.7) (end 159.55 115.7) (width 1) (layer B.Cu) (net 7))
 (segment (start 159.55 115.7) (end 164.25 111) (width 1) (layer B.Cu) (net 7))
 (segment (start 136 110) (end 136 113.25) (width 1) (layer F.Cu) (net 7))
 (segment (start 144.975 114.275) (end 144.975 111.675) (width 1) (layer F.Cu) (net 7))
 (segment (start 143.75 115.25) (end 144.975 114.275) (width 1) (layer F.Cu) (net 7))
 (segment (start 138.25 115.25) (end 143.75 115.25) (width 1) (layer F.Cu) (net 7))
 (segment (start 136 113.25) (end 138.25 115.25) (width 1) (layer F.Cu) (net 7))
 (segment (start 144.975 112.95) (end 144.975 111.675) (width 1) (layer B.Cu) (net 7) (status 20))
 (segment (start 158.25 115.7) (end 147.725 115.7) (width 1) (layer B.Cu) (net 7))
 (segment (start 169.2 111) (end 164.25 111) (width 1) (layer B.Cu) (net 7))
 (segment (start 147.725 115.7) (end 144.975 112.95) (width 1) (layer B.Cu) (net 7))
 (segment (start 136 110) (end 136 110.075) (width 1) (layer B.Cu) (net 7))
 (segment (start 169 111) (end 169.2 111) (width 1) (layer F.Cu) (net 7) (status 30))
 (segment (start 128 102) (end 128 104) (width 1) (layer B.Cu) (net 7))
 (segment (start 130 108) (end 132 110) (width 1) (layer B.Cu) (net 7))
 (segment (start 130 106) (end 130 108) (width 1) (layer B.Cu) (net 7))
 (segment (start 128 104) (end 130 106) (width 1) (layer B.Cu) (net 7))
 (segment (start 124 101.38) (end 127.38 101.38) (width 1) (layer B.Cu) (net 7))
 (segment (start 127.38 101.38) (end 128 102) (width 1) (layer B.Cu) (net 7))
 (segment (start 132 110) (end 136 110) (width 1) (layer B.Cu) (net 7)))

